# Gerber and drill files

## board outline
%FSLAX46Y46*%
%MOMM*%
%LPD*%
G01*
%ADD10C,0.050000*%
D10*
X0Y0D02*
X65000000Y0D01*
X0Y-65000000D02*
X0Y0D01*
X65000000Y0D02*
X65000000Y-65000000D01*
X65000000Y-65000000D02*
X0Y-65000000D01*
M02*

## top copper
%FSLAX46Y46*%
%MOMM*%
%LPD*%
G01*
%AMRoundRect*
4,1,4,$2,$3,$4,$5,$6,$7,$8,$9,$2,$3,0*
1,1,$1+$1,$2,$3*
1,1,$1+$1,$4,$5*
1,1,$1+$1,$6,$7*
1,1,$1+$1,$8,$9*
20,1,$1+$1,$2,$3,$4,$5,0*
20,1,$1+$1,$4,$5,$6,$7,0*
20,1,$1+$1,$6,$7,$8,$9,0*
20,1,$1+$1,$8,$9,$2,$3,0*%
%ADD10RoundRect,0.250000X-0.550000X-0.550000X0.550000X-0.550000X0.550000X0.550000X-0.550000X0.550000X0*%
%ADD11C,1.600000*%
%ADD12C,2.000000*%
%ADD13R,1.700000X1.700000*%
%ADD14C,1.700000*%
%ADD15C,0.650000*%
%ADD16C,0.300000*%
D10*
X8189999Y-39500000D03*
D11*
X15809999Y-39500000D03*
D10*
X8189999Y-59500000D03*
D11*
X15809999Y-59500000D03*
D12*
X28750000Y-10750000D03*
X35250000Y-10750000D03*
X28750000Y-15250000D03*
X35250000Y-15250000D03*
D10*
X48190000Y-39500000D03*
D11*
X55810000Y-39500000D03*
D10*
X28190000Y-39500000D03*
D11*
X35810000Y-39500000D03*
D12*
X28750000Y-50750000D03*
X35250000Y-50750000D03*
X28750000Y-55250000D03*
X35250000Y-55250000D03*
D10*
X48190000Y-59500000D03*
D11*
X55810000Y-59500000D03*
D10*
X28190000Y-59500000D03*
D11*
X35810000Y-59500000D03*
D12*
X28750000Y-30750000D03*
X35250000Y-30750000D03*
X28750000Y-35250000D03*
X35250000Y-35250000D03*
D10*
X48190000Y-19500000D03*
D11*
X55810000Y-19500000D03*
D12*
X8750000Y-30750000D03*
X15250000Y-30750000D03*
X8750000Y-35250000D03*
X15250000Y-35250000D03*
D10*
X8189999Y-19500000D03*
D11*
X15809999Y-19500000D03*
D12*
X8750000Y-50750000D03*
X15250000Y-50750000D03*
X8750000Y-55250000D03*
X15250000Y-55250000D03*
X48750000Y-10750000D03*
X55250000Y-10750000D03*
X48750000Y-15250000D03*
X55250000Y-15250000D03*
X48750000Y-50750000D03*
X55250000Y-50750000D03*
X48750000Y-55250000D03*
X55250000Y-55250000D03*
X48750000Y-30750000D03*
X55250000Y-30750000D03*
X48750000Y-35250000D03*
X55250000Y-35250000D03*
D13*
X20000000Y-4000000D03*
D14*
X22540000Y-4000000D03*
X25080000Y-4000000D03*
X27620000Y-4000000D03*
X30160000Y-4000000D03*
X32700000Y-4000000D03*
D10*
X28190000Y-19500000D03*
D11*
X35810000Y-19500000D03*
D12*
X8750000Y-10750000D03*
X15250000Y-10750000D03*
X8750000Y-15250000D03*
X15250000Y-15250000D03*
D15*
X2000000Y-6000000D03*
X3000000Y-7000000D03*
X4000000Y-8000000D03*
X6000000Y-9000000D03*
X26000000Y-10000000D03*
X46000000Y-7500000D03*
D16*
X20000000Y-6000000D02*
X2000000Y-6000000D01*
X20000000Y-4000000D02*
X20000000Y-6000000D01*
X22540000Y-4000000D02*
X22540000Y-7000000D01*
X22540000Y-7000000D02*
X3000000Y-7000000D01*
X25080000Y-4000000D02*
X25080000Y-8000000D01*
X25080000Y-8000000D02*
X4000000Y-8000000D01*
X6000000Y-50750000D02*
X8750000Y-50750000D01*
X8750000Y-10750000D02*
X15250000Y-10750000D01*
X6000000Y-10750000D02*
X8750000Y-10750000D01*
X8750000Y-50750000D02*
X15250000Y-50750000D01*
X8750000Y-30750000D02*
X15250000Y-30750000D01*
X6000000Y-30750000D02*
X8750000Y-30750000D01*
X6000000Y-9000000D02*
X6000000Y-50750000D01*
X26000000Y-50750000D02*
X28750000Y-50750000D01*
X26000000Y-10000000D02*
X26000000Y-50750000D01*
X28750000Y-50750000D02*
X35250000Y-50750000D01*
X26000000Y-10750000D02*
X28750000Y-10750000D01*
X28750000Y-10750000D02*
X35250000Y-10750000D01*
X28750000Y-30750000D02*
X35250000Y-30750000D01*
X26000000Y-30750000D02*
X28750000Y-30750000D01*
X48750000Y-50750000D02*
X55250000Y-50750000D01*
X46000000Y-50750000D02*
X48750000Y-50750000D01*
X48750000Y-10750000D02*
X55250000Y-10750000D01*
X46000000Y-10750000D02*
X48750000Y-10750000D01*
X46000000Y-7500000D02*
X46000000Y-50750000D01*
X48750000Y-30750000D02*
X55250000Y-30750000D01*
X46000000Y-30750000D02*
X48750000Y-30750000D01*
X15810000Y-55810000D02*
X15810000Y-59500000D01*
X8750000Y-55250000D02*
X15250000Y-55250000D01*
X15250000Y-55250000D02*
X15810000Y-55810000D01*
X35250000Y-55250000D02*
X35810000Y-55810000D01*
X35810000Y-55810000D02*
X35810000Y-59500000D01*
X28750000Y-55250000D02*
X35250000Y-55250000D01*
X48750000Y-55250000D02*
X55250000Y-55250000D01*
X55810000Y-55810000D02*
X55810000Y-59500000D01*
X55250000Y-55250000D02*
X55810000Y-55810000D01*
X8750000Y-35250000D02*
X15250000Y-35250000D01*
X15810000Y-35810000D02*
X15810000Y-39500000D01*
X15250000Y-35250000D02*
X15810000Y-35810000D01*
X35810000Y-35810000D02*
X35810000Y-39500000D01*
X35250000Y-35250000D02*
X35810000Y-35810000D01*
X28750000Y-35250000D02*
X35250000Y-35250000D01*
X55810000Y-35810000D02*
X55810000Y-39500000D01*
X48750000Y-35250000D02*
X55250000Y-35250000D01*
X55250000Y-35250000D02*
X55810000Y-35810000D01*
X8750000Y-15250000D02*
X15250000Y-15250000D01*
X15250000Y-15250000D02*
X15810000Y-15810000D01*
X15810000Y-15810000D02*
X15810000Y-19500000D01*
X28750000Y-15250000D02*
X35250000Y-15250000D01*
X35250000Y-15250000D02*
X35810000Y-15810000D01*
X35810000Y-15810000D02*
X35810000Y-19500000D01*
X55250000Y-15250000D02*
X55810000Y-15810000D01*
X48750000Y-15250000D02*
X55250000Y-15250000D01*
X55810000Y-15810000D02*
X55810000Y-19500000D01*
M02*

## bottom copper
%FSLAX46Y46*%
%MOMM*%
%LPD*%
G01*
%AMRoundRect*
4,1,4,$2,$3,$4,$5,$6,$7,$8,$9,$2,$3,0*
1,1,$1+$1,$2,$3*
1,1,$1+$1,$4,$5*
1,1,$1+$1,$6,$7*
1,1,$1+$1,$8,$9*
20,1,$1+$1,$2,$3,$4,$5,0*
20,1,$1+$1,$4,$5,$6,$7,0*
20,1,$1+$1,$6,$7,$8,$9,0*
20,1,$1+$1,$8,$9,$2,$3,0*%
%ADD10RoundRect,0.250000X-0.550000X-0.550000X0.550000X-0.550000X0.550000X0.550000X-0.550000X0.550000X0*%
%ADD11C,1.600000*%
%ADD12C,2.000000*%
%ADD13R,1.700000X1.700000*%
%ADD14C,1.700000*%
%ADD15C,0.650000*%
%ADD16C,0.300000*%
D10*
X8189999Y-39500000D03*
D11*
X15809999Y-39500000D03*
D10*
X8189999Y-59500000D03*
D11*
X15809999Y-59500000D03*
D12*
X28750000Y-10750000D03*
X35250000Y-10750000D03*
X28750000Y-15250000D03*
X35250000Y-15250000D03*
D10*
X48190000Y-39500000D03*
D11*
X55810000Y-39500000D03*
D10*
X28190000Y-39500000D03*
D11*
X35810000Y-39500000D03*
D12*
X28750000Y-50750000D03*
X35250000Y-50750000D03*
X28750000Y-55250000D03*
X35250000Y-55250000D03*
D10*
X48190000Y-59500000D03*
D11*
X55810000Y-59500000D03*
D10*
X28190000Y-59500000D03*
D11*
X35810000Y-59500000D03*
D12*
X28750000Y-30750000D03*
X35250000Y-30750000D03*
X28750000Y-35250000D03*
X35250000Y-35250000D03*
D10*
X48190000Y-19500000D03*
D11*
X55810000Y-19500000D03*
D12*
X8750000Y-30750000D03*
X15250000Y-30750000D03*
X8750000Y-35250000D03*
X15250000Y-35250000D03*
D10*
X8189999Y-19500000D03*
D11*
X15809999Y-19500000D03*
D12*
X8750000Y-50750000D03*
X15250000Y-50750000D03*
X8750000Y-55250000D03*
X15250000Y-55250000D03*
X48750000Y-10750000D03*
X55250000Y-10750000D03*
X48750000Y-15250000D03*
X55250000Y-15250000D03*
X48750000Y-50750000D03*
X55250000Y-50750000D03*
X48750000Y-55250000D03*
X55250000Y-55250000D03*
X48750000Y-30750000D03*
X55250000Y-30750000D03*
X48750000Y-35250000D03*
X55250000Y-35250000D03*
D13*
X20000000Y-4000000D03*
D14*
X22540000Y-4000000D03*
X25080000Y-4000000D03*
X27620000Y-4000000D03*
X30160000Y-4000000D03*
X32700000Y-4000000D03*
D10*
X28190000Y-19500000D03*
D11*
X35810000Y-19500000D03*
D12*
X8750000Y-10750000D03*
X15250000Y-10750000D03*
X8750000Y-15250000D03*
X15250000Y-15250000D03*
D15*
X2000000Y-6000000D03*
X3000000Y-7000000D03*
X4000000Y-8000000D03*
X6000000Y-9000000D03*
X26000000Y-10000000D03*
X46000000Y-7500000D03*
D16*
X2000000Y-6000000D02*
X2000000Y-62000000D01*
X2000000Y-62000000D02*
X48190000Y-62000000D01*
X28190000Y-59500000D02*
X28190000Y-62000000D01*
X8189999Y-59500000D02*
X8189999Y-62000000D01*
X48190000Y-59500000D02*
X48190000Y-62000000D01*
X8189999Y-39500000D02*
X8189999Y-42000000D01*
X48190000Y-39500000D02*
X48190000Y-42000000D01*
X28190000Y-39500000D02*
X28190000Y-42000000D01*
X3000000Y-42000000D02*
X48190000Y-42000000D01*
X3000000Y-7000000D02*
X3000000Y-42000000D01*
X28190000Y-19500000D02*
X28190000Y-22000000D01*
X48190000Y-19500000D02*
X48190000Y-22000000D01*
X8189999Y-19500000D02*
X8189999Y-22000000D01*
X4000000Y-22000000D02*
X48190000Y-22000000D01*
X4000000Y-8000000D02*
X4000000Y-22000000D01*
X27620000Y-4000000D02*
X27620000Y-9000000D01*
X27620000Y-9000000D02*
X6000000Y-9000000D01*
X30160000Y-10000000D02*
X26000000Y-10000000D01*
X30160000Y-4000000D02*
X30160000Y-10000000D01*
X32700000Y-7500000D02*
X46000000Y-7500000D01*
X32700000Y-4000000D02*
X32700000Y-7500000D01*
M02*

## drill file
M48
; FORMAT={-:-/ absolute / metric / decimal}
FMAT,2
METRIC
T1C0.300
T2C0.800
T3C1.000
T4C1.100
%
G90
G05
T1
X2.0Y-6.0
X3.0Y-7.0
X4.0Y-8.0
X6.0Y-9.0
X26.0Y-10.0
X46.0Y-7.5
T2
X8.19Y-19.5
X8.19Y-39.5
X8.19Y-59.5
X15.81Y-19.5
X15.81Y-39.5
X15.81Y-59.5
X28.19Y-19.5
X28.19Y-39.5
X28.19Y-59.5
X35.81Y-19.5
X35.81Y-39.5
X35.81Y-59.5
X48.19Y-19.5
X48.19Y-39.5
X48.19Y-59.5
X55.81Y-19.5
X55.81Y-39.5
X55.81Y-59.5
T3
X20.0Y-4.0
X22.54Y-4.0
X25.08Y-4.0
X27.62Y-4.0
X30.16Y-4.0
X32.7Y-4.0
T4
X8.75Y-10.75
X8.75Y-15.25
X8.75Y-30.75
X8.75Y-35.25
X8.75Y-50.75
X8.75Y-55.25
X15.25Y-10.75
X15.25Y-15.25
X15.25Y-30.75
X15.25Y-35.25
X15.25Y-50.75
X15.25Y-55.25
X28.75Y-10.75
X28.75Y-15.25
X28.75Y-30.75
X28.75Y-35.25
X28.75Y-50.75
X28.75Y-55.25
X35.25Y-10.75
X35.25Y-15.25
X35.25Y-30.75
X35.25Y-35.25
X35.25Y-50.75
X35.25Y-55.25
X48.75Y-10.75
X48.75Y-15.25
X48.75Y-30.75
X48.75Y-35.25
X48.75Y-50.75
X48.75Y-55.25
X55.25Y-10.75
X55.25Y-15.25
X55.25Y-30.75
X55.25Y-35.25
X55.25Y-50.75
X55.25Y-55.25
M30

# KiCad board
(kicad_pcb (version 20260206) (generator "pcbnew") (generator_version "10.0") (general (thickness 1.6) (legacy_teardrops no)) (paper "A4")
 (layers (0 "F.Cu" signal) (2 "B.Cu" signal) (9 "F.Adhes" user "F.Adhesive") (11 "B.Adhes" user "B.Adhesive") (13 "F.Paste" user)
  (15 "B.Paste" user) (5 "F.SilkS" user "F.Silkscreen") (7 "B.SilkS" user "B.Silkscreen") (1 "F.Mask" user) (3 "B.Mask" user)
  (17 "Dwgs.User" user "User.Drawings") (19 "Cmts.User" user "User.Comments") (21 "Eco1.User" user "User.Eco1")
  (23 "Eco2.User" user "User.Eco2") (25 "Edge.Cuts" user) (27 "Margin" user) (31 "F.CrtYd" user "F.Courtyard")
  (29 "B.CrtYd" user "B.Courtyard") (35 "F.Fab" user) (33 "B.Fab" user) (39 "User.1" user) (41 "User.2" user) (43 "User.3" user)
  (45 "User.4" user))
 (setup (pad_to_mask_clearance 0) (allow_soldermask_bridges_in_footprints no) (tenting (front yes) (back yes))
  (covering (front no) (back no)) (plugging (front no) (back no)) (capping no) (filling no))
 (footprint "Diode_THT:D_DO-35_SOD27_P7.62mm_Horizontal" (layer "F.Cu") (at 8.189999 39.5)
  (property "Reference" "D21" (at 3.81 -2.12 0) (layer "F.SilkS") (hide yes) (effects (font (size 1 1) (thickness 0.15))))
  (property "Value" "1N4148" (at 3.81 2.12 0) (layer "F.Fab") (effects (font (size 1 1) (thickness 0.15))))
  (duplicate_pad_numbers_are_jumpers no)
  (pad "1" thru_hole roundrect (at 0 0) (size 1.6 1.6) (drill 0.8) (layers "*.Cu" "*.Mask") (remove_unused_layers no)
   (roundrect_rratio 0.15625) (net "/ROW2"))
  (pad "2" thru_hole circle (at 7.62 0) (size 1.6 1.6) (drill 0.8) (layers "*.Cu" "*.Mask") (remove_unused_layers no) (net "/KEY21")))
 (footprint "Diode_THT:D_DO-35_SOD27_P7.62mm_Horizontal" (layer "F.Cu") (at 8.189999 59.5)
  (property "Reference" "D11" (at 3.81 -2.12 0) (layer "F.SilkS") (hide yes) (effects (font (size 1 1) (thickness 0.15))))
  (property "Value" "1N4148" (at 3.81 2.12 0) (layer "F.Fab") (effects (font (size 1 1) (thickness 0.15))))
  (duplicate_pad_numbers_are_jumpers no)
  (pad "1" thru_hole roundrect (at 0 0) (size 1.6 1.6) (drill 0.8) (layers "*.Cu" "*.Mask") (remove_unused_layers no)
   (roundrect_rratio 0.15625) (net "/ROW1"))
  (pad "2" thru_hole circle (at 7.62 0) (size 1.6 1.6) (drill 0.8) (layers "*.Cu" "*.Mask") (remove_unused_layers no) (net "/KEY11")))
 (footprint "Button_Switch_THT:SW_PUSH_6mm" (layer "F.Cu") (at 28.75 10.75)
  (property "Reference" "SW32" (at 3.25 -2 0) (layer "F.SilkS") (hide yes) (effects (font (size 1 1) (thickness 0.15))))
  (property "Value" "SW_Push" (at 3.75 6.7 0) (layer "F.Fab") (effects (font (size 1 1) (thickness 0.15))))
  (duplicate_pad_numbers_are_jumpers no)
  (pad "1" thru_hole circle (at 0 0 90) (size 2 2) (drill 1.1) (layers "*.Cu" "*.Mask") (remove_unused_layers no) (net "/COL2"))
  (pad "1" thru_hole circle (at 6.5 0 90) (size 2 2) (drill 1.1) (layers "*.Cu" "*.Mask") (remove_unused_layers no) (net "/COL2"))
  (pad "2" thru_hole circle (at 0 4.5 90) (size 2 2) (drill 1.1) (layers "*.Cu" "*.Mask") (remove_unused_layers no) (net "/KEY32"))
  (pad "2" thru_hole circle (at 6.5 4.5 90) (size 2 2) (drill 1.1) (layers "*.Cu" "*.Mask") (remove_unused_layers no) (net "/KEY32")))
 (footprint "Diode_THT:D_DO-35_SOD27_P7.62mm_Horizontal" (layer "F.Cu") (at 48.19 39.5)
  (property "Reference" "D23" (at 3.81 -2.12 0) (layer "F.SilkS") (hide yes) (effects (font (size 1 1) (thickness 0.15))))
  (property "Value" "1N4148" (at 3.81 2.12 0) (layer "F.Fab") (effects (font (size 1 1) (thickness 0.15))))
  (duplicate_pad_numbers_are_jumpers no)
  (pad "1" thru_hole roundrect (at 0 0) (size 1.6 1.6) (drill 0.8) (layers "*.Cu" "*.Mask") (remove_unused_layers no)
   (roundrect_rratio 0.15625) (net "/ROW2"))
  (pad "2" thru_hole circle (at 7.62 0) (size 1.6 1.6) (drill 0.8) (layers "*.Cu" "*.Mask") (remove_unused_layers no) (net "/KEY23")))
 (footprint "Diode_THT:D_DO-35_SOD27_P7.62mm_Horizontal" (layer "F.Cu") (at 28.19 39.5)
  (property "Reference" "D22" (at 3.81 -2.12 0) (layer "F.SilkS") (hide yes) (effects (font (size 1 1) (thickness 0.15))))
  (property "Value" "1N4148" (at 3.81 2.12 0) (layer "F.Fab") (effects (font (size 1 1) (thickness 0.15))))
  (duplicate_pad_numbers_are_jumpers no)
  (pad "1" thru_hole roundrect (at 0 0) (size 1.6 1.6) (drill 0.8) (layers "*.Cu" "*.Mask") (remove_unused_layers no)
   (roundrect_rratio 0.15625) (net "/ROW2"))
  (pad "2" thru_hole circle (at 7.62 0) (size 1.6 1.6) (drill 0.8) (layers "*.Cu" "*.Mask") (remove_unused_layers no) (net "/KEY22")))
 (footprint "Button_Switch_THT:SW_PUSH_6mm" (layer "F.Cu") (at 28.75 50.75)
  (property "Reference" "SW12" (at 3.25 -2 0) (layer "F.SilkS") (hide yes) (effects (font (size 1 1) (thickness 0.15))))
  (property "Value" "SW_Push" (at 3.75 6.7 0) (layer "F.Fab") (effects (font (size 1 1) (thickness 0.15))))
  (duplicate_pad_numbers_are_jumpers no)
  (pad "1" thru_hole circle (at 0 0 90) (size 2 2) (drill 1.1) (layers "*.Cu" "*.Mask") (remove_unused_layers no) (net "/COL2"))
  (pad "1" thru_hole circle (at 6.5 0 90) (size 2 2) (drill 1.1) (layers "*.Cu" "*.Mask") (remove_unused_layers no) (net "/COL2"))
  (pad "2" thru_hole circle (at 0 4.5 90) (size 2 2) (drill 1.1) (layers "*.Cu" "*.Mask") (remove_unused_layers no) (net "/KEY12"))
  (pad "2" thru_hole circle (at 6.5 4.5 90) (size 2 2) (drill 1.1) (layers "*.Cu" "*.Mask") (remove_unused_layers no) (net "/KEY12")))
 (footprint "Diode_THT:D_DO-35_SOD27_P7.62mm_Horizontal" (layer "F.Cu") (at 48.19 59.5)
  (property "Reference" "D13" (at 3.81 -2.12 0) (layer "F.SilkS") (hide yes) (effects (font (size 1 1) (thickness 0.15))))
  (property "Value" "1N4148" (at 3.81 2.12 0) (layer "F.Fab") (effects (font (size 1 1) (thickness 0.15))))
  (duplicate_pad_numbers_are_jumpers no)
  (pad "1" thru_hole roundrect (at 0 0) (size 1.6 1.6) (drill 0.8) (layers "*.Cu" "*.Mask") (remove_unused_layers no)
   (roundrect_rratio 0.15625) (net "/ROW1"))
  (pad "2" thru_hole circle (at 7.62 0) (size 1.6 1.6) (drill 0.8) (layers "*.Cu" "*.Mask") (remove_unused_layers no) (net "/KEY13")))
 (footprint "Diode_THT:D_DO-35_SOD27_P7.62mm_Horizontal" (layer "F.Cu") (at 28.19 59.5)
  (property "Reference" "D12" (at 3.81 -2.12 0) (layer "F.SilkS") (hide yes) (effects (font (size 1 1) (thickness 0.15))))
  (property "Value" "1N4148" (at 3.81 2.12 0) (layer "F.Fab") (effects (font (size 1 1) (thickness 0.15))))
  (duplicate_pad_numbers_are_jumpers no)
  (pad "1" thru_hole roundrect (at 0 0) (size 1.6 1.6) (drill 0.8) (layers "*.Cu" "*.Mask") (remove_unused_layers no)
   (roundrect_rratio 0.15625) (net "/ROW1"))
  (pad "2" thru_hole circle (at 7.62 0) (size 1.6 1.6) (drill 0.8) (layers "*.Cu" "*.Mask") (remove_unused_layers no) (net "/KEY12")))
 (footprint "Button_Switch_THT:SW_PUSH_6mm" (layer "F.Cu") (at 28.75 30.75)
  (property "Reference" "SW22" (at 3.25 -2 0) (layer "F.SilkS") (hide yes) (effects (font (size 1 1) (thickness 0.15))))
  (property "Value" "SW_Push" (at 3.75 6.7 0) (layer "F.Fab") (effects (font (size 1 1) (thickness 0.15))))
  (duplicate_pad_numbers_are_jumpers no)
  (pad "1" thru_hole circle (at 0 0 90) (size 2 2) (drill 1.1) (layers "*.Cu" "*.Mask") (remove_unused_layers no) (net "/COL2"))
  (pad "1" thru_hole circle (at 6.5 0 90) (size 2 2) (drill 1.1) (layers "*.Cu" "*.Mask") (remove_unused_layers no) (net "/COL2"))
  (pad "2" thru_hole circle (at 0 4.5 90) (size 2 2) (drill 1.1) (layers "*.Cu" "*.Mask") (remove_unused_layers no) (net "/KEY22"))
  (pad "2" thru_hole circle (at 6.5 4.5 90) (size 2 2) (drill 1.1) (layers "*.Cu" "*.Mask") (remove_unused_layers no) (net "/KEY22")))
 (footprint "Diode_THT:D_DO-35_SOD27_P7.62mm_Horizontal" (layer "F.Cu") (at 48.19 19.5)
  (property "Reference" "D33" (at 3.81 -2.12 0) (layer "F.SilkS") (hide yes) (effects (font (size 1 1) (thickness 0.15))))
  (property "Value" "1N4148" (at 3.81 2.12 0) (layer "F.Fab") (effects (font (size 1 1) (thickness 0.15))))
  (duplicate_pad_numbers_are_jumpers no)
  (pad "1" thru_hole roundrect (at 0 0) (size 1.6 1.6) (drill 0.8) (layers "*.Cu" "*.Mask") (remove_unused_layers no)
   (roundrect_rratio 0.15625) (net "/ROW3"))
  (pad "2" thru_hole circle (at 7.62 0) (size 1.6 1.6) (drill 0.8) (layers "*.Cu" "*.Mask") (remove_unused_layers no) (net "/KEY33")))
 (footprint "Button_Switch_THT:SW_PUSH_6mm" (layer "F.Cu") (at 8.75 30.75)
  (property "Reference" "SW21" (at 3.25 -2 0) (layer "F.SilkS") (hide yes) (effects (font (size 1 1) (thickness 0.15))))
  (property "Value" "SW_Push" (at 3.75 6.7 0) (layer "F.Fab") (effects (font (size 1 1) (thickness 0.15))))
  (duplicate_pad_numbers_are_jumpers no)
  (pad "1" thru_hole circle (at 0 0 90) (size 2 2) (drill 1.1) (layers "*.Cu" "*.Mask") (remove_unused_layers no) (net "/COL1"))
  (pad "1" thru_hole circle (at 6.5 0 90) (size 2 2) (drill 1.1) (layers "*.Cu" "*.Mask") (remove_unused_layers no) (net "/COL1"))
  (pad "2" thru_hole circle (at 0 4.5 90) (size 2 2) (drill 1.1) (layers "*.Cu" "*.Mask") (remove_unused_layers no) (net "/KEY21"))
  (pad "2" thru_hole circle (at 6.5 4.5 90) (size 2 2) (drill 1.1) (layers "*.Cu" "*.Mask") (remove_unused_layers no) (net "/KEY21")))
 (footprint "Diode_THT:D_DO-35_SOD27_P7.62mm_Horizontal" (layer "F.Cu") (at 8.189999 19.5)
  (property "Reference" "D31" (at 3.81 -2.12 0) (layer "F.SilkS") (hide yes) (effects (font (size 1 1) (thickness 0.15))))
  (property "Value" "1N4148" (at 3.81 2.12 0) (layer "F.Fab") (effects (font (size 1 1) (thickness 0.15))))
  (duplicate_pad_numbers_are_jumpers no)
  (pad "1" thru_hole roundrect (at 0 0) (size 1.6 1.6) (drill 0.8) (layers "*.Cu" "*.Mask") (remove_unused_layers no)
   (roundrect_rratio 0.15625) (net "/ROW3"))
  (pad "2" thru_hole circle (at 7.62 0) (size 1.6 1.6) (drill 0.8) (layers "*.Cu" "*.Mask") (remove_unused_layers no) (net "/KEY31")))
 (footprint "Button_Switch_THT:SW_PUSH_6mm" (layer "F.Cu") (at 8.75 50.75)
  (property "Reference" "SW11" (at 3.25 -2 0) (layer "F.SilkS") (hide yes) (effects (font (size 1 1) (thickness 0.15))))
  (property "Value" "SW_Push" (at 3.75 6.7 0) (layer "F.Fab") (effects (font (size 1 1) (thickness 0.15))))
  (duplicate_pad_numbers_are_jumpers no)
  (pad "1" thru_hole circle (at 0 0 90) (size 2 2) (drill 1.1) (layers "*.Cu" "*.Mask") (remove_unused_layers no) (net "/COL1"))
  (pad "1" thru_hole circle (at 6.5 0 90) (size 2 2) (drill 1.1) (layers "*.Cu" "*.Mask") (remove_unused_layers no) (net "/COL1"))
  (pad "2" thru_hole circle (at 0 4.5 90) (size 2 2) (drill 1.1) (layers "*.Cu" "*.Mask") (remove_unused_layers no) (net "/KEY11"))
  (pad "2" thru_hole circle (at 6.5 4.5 90) (size 2 2) (drill 1.1) (layers "*.Cu" "*.Mask") (remove_unused_layers no) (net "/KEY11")))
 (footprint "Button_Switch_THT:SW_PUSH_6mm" (layer "F.Cu") (at 48.75 10.75)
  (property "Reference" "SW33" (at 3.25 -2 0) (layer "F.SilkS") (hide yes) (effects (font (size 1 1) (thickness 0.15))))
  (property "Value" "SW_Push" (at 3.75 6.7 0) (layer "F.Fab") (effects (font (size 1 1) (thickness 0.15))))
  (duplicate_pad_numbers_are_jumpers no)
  (pad "1" thru_hole circle (at 0 0 90) (size 2 2) (drill 1.1) (layers "*.Cu" "*.Mask") (remove_unused_layers no) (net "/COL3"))
  (pad "1" thru_hole circle (at 6.5 0 90) (size 2 2) (drill 1.1) (layers "*.Cu" "*.Mask") (remove_unused_layers no) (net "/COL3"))
  (pad "2" thru_hole circle (at 0 4.5 90) (size 2 2) (drill 1.1) (layers "*.Cu" "*.Mask") (remove_unused_layers no) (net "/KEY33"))
  (pad "2" thru_hole circle (at 6.5 4.5 90) (size 2 2) (drill 1.1) (layers "*.Cu" "*.Mask") (remove_unused_layers no) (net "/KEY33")))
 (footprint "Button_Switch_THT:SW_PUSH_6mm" (layer "F.Cu") (at 48.75 50.75)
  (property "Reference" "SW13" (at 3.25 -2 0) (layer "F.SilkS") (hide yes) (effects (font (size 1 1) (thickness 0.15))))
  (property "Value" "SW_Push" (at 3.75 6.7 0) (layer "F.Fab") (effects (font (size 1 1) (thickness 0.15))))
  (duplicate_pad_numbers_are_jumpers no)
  (pad "1" thru_hole circle (at 0 0 90) (size 2 2) (drill 1.1) (layers "*.Cu" "*.Mask") (remove_unused_layers no) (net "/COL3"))
  (pad "1" thru_hole circle (at 6.5 0 90) (size 2 2) (drill 1.1) (layers "*.Cu" "*.Mask") (remove_unused_layers no) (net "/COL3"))
  (pad "2" thru_hole circle (at 0 4.5 90) (size 2 2) (drill 1.1) (layers "*.Cu" "*.Mask") (remove_unused_layers no) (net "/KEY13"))
  (pad "2" thru_hole circle (at 6.5 4.5 90) (size 2 2) (drill 1.1) (layers "*.Cu" "*.Mask") (remove_unused_layers no) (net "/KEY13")))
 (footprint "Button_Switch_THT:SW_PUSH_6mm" (layer "F.Cu") (at 48.75 30.75)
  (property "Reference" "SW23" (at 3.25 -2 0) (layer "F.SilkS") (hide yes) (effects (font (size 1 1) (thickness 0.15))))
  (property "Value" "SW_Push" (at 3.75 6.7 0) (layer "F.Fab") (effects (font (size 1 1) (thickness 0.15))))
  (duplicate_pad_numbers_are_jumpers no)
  (pad "1" thru_hole circle (at 0 0 90) (size 2 2) (drill 1.1) (layers "*.Cu" "*.Mask") (remove_unused_layers no) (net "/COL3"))
  (pad "1" thru_hole circle (at 6.5 0 90) (size 2 2) (drill 1.1) (layers "*.Cu" "*.Mask") (remove_unused_layers no) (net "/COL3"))
  (pad "2" thru_hole circle (at 0 4.5 90) (size 2 2) (drill 1.1) (layers "*.Cu" "*.Mask") (remove_unused_layers no) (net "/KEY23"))
  (pad "2" thru_hole circle (at 6.5 4.5 90) (size 2 2) (drill 1.1) (layers "*.Cu" "*.Mask") (remove_unused_layers no) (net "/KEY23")))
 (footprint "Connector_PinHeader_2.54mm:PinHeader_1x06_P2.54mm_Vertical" (layer "F.Cu") (at 20 4 90)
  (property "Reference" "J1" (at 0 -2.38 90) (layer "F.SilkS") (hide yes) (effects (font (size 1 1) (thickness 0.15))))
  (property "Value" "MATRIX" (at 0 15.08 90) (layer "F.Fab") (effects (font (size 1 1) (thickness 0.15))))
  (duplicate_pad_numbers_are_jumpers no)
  (pad "1" thru_hole rect (at 0 0 90) (size 1.7 1.7) (drill 1) (layers "*.Cu" "*.Mask") (remove_unused_layers no) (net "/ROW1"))
  (pad "2" thru_hole circle (at 0 2.54 90) (size 1.7 1.7) (drill 1) (layers "*.Cu" "*.Mask") (remove_unused_layers no) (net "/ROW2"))
  (pad "3" thru_hole circle (at 0 5.08 90) (size 1.7 1.7) (drill 1) (layers "*.Cu" "*.Mask") (remove_unused_layers no) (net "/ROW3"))
  (pad "4" thru_hole circle (at 0 7.62 90) (size 1.7 1.7) (drill 1) (layers "*.Cu" "*.Mask") (remove_unused_layers no) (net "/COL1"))
  (pad "5" thru_hole circle (at 0 10.16 90) (size 1.7 1.7) (drill 1) (layers "*.Cu" "*.Mask") (remove_unused_layers no) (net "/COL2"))
  (pad "6" thru_hole circle (at 0 12.7 90) (size 1.7 1.7) (drill 1) (layers "*.Cu" "*.Mask") (remove_unused_layers no) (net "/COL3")))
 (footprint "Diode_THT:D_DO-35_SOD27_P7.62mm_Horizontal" (layer "F.Cu") (at 28.19 19.5)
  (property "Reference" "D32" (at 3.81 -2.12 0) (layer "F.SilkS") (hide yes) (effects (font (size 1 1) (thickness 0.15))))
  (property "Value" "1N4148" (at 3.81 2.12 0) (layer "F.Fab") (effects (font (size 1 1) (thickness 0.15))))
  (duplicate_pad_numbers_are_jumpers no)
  (pad "1" thru_hole roundrect (at 0 0) (size 1.6 1.6) (drill 0.8) (layers "*.Cu" "*.Mask") (remove_unused_layers no)
   (roundrect_rratio 0.15625) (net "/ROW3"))
  (pad "2" thru_hole circle (at 7.62 0) (size 1.6 1.6) (drill 0.8) (layers "*.Cu" "*.Mask") (remove_unused_layers no) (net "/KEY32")))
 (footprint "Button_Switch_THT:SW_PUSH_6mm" (layer "F.Cu") (at 8.75 10.75)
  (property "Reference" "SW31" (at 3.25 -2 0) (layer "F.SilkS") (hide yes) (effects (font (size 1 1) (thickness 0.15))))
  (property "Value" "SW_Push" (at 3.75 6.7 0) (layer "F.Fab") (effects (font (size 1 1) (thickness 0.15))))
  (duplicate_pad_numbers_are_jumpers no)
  (pad "1" thru_hole circle (at 0 0 90) (size 2 2) (drill 1.1) (layers "*.Cu" "*.Mask") (remove_unused_layers no) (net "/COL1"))
  (pad "1" thru_hole circle (at 6.5 0 90) (size 2 2) (drill 1.1) (layers "*.Cu" "*.Mask") (remove_unused_layers no) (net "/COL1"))
  (pad "2" thru_hole circle (at 0 4.5 90) (size 2 2) (drill 1.1) (layers "*.Cu" "*.Mask") (remove_unused_layers no) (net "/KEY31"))
  (pad "2" thru_hole circle (at 6.5 4.5 90) (size 2 2) (drill 1.1) (layers "*.Cu" "*.Mask") (remove_unused_layers no) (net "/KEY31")))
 (gr_line (start 0 0) (end 65 0) (stroke (width 0.05) (type default)) (layer "Edge.Cuts"))
 (gr_line (start 0 65) (end 0 0) (stroke (width 0.05) (type default)) (layer "Edge.Cuts"))
 (gr_line (start 65 0) (end 65 65) (stroke (width 0.05) (type default)) (layer "Edge.Cuts"))
 (gr_line (start 65 65) (end 0 65) (stroke (width 0.05) (type default)) (layer "Edge.Cuts"))
 (segment (start 20 6) (end 2 6) (width 0.3) (layer "F.Cu") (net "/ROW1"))
 (segment (start 20 4) (end 20 6) (width 0.3) (layer "F.Cu") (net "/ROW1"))
 (via (at 2 6) (size 0.65) (drill 0.3) (layers "F.Cu" "B.Cu") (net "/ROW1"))
 (segment (start 2 6) (end 2 62) (width 0.3) (layer "B.Cu") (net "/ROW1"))
 (segment (start 2 62) (end 48.19 62) (width 0.3) (layer "B.Cu") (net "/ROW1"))
 (segment (start 28.19 59.5) (end 28.19 62) (width 0.3) (layer "B.Cu") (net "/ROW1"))
 (segment (start 8.189999 59.5) (end 8.189999 62) (width 0.3) (layer "B.Cu") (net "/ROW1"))
 (segment (start 48.19 59.5) (end 48.19 62) (width 0.3) (layer "B.Cu") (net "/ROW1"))
 (segment (start 22.54 4) (end 22.54 7) (width 0.3) (layer "F.Cu") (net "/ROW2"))
 (segment (start 22.54 7) (end 3 7) (width 0.3) (layer "F.Cu") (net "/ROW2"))
 (via (at 3 7) (size 0.65) (drill 0.3) (layers "F.Cu" "B.Cu") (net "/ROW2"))
 (segment (start 8.189999 39.5) (end 8.189999 42) (width 0.3) (layer "B.Cu") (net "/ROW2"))
 (segment (start 48.19 39.5) (end 48.19 42) (width 0.3) (layer "B.Cu") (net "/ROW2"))
 (segment (start 28.19 39.5) (end 28.19 42) (width 0.3) (layer "B.Cu") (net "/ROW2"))
 (segment (start 3 42) (end 48.19 42) (width 0.3) (layer "B.Cu") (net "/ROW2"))
 (segment (start 3 7) (end 3 42) (width 0.3) (layer "B.Cu") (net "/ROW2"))
 (segment (start 25.08 4) (end 25.08 8) (width 0.3) (layer "F.Cu") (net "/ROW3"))
 (segment (start 25.08 8) (end 4 8) (width 0.3) (layer "F.Cu") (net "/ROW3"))
 (via (at 4 8) (size 0.65) (drill 0.3) (layers "F.Cu" "B.Cu") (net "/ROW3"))
 (segment (start 28.19 19.5) (end 28.19 22) (width 0.3) (layer "B.Cu") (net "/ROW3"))
 (segment (start 48.19 19.5) (end 48.19 22) (width 0.3) (layer "B.Cu") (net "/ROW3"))
 (segment (start 8.189999 19.5) (end 8.189999 22) (width 0.3) (layer "B.Cu") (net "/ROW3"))
 (segment (start 4 22) (end 48.19 22) (width 0.3) (layer "B.Cu") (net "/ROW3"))
 (segment (start 4 8) (end 4 22) (width 0.3) (layer "B.Cu") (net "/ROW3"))
 (segment (start 6 50.75) (end 8.75 50.75) (width 0.3) (layer "F.Cu") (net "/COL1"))
 (segment (start 8.75 10.75) (end 15.25 10.75) (width 0.3) (layer "F.Cu") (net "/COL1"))
 (segment (start 6 10.75) (end 8.75 10.75) (width 0.3) (layer "F.Cu") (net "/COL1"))
 (segment (start 8.75 50.75) (end 15.25 50.75) (width 0.3) (layer "F.Cu") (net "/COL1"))
 (segment (start 8.75 30.75) (end 15.25 30.75) (width 0.3) (layer "F.Cu") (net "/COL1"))
 (segment (start 6 30.75) (end 8.75 30.75) (width 0.3) (layer "F.Cu") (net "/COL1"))
 (segment (start 6 9) (end 6 50.75) (width 0.3) (layer "F.Cu") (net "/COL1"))
 (via (at 6 9) (size 0.65) (drill 0.3) (layers "F.Cu" "B.Cu") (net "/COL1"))
 (segment (start 27.62 4) (end 27.62 9) (width 0.3) (layer "B.Cu") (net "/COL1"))
 (segment (start 27.62 9) (end 6 9) (width 0.3) (layer "B.Cu") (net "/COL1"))
 (segment (start 26 50.75) (end 28.75 50.75) (width 0.3) (layer "F.Cu") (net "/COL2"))
 (segment (start 26 10) (end 26 50.75) (width 0.3) (layer "F.Cu") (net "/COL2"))
 (segment (start 28.75 50.75) (end 35.25 50.75) (width 0.3) (layer "F.Cu") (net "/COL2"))
 (segment (start 26 10.75) (end 28.75 10.75) (width 0.3) (layer "F.Cu") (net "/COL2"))
 (segment (start 28.75 10.75) (end 35.25 10.75) (width 0.3) (layer "F.Cu") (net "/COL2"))
 (segment (start 28.75 30.75) (end 35.25 30.75) (width 0.3) (layer "F.Cu") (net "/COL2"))
 (segment (start 26 30.75) (end 28.75 30.75) (width 0.3) (layer "F.Cu") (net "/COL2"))
 (via (at 26 10) (size 0.65) (drill 0.3) (layers "F.Cu" "B.Cu") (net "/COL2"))
 (segment (start 30.16 10) (end 26 10) (width 0.3) (layer "B.Cu") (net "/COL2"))
 (segment (start 30.16 4) (end 30.16 10) (width 0.3) (layer "B.Cu") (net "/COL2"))
 (segment (start 48.75 50.75) (end 55.25 50.75) (width 0.3) (layer "F.Cu") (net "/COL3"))
 (segment (start 46 50.75) (end 48.75 50.75) (width 0.3) (layer "F.Cu") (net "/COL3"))
 (segment (start 48.75 10.75) (end 55.25 10.75) (width 0.3) (layer "F.Cu") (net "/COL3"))
 (segment (start 46 10.75) (end 48.75 10.75) (width 0.3) (layer "F.Cu") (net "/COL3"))
 (segment (start 46 7.5) (end 46 50.75) (width 0.3) (layer "F.Cu") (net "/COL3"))
 (segment (start 48.75 30.75) (end 55.25 30.75) (width 0.3) (layer "F.Cu") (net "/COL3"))
 (segment (start 46 30.75) (end 48.75 30.75) (width 0.3) (layer "F.Cu") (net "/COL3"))
 (via (at 46 7.5) (size 0.65) (drill 0.3) (layers "F.Cu" "B.Cu") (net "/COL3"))
 (segment (start 32.7 7.5) (end 46 7.5) (width 0.3) (layer "B.Cu") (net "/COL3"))
 (segment (start 32.7 4) (end 32.7 7.5) (width 0.3) (layer "B.Cu") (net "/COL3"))
 (segment (start 15.81 55.81) (end 15.81 59.5) (width 0.3) (layer "F.Cu") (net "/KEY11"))
 (segment (start 8.75 55.25) (end 15.25 55.25) (width 0.3) (layer "F.Cu") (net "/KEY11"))
 (segment (start 15.25 55.25) (end 15.81 55.81) (width 0.3) (layer "F.Cu") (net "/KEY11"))
 (segment (start 35.25 55.25) (end 35.81 55.81) (width 0.3) (layer "F.Cu") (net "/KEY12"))
 (segment (start 35.81 55.81) (end 35.81 59.5) (width 0.3) (layer "F.Cu") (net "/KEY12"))
 (segment (start 28.75 55.25) (end 35.25 55.25) (width 0.3) (layer "F.Cu") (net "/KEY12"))
 (segment (start 48.75 55.25) (end 55.25 55.25) (width 0.3) (layer "F.Cu") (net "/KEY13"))
 (segment (start 55.81 55.81) (end 55.81 59.5) (width 0.3) (layer "F.Cu") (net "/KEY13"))
 (segment (start 55.25 55.25) (end 55.81 55.81) (width 0.3) (layer "F.Cu") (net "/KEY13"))
 (segment (start 8.75 35.25) (end 15.25 35.25) (width 0.3) (layer "F.Cu") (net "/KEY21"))
 (segment (start 15.81 35.81) (end 15.81 39.5) (width 0.3) (layer "F.Cu") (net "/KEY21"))
 (segment (start 15.25 35.25) (end 15.81 35.81) (width 0.3) (layer "F.Cu") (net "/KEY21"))
 (segment (start 35.81 35.81) (end 35.81 39.5) (width 0.3) (layer "F.Cu") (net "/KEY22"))
 (segment (start 35.25 35.25) (end 35.81 35.81) (width 0.3) (layer "F.Cu") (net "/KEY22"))
 (segment (start 28.75 35.25) (end 35.25 35.25) (width 0.3) (layer "F.Cu") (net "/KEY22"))
 (segment (start 55.81 35.81) (end 55.81 39.5) (width 0.3) (layer "F.Cu") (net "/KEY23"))
 (segment (start 48.75 35.25) (end 55.25 35.25) (width 0.3) (layer "F.Cu") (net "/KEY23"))
 (segment (start 55.25 35.25) (end 55.81 35.81) (width 0.3) (layer "F.Cu") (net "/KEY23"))
 (segment (start 8.75 15.25) (end 15.25 15.25) (width 0.3) (layer "F.Cu") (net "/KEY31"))
 (segment (start 15.25 15.25) (end 15.81 15.81) (width 0.3) (layer "F.Cu") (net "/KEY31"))
 (segment (start 15.81 15.81) (end 15.81 19.5) (width 0.3) (layer "F.Cu") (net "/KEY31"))
 (segment (start 28.75 15.25) (end 35.25 15.25) (width 0.3) (layer "F.Cu") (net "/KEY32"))
 (segment (start 35.25 15.25) (end 35.81 15.81) (width 0.3) (layer "F.Cu") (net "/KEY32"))
 (segment (start 35.81 15.81) (end 35.81 19.5) (width 0.3) (layer "F.Cu") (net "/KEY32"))
 (segment (start 55.25 15.25) (end 55.81 15.81) (width 0.3) (layer "F.Cu") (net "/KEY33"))
 (segment (start 48.75 15.25) (end 55.25 15.25) (width 0.3) (layer "F.Cu") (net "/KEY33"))
 (segment (start 55.81 15.81) (end 55.81 19.5) (width 0.3) (layer "F.Cu") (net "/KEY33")))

